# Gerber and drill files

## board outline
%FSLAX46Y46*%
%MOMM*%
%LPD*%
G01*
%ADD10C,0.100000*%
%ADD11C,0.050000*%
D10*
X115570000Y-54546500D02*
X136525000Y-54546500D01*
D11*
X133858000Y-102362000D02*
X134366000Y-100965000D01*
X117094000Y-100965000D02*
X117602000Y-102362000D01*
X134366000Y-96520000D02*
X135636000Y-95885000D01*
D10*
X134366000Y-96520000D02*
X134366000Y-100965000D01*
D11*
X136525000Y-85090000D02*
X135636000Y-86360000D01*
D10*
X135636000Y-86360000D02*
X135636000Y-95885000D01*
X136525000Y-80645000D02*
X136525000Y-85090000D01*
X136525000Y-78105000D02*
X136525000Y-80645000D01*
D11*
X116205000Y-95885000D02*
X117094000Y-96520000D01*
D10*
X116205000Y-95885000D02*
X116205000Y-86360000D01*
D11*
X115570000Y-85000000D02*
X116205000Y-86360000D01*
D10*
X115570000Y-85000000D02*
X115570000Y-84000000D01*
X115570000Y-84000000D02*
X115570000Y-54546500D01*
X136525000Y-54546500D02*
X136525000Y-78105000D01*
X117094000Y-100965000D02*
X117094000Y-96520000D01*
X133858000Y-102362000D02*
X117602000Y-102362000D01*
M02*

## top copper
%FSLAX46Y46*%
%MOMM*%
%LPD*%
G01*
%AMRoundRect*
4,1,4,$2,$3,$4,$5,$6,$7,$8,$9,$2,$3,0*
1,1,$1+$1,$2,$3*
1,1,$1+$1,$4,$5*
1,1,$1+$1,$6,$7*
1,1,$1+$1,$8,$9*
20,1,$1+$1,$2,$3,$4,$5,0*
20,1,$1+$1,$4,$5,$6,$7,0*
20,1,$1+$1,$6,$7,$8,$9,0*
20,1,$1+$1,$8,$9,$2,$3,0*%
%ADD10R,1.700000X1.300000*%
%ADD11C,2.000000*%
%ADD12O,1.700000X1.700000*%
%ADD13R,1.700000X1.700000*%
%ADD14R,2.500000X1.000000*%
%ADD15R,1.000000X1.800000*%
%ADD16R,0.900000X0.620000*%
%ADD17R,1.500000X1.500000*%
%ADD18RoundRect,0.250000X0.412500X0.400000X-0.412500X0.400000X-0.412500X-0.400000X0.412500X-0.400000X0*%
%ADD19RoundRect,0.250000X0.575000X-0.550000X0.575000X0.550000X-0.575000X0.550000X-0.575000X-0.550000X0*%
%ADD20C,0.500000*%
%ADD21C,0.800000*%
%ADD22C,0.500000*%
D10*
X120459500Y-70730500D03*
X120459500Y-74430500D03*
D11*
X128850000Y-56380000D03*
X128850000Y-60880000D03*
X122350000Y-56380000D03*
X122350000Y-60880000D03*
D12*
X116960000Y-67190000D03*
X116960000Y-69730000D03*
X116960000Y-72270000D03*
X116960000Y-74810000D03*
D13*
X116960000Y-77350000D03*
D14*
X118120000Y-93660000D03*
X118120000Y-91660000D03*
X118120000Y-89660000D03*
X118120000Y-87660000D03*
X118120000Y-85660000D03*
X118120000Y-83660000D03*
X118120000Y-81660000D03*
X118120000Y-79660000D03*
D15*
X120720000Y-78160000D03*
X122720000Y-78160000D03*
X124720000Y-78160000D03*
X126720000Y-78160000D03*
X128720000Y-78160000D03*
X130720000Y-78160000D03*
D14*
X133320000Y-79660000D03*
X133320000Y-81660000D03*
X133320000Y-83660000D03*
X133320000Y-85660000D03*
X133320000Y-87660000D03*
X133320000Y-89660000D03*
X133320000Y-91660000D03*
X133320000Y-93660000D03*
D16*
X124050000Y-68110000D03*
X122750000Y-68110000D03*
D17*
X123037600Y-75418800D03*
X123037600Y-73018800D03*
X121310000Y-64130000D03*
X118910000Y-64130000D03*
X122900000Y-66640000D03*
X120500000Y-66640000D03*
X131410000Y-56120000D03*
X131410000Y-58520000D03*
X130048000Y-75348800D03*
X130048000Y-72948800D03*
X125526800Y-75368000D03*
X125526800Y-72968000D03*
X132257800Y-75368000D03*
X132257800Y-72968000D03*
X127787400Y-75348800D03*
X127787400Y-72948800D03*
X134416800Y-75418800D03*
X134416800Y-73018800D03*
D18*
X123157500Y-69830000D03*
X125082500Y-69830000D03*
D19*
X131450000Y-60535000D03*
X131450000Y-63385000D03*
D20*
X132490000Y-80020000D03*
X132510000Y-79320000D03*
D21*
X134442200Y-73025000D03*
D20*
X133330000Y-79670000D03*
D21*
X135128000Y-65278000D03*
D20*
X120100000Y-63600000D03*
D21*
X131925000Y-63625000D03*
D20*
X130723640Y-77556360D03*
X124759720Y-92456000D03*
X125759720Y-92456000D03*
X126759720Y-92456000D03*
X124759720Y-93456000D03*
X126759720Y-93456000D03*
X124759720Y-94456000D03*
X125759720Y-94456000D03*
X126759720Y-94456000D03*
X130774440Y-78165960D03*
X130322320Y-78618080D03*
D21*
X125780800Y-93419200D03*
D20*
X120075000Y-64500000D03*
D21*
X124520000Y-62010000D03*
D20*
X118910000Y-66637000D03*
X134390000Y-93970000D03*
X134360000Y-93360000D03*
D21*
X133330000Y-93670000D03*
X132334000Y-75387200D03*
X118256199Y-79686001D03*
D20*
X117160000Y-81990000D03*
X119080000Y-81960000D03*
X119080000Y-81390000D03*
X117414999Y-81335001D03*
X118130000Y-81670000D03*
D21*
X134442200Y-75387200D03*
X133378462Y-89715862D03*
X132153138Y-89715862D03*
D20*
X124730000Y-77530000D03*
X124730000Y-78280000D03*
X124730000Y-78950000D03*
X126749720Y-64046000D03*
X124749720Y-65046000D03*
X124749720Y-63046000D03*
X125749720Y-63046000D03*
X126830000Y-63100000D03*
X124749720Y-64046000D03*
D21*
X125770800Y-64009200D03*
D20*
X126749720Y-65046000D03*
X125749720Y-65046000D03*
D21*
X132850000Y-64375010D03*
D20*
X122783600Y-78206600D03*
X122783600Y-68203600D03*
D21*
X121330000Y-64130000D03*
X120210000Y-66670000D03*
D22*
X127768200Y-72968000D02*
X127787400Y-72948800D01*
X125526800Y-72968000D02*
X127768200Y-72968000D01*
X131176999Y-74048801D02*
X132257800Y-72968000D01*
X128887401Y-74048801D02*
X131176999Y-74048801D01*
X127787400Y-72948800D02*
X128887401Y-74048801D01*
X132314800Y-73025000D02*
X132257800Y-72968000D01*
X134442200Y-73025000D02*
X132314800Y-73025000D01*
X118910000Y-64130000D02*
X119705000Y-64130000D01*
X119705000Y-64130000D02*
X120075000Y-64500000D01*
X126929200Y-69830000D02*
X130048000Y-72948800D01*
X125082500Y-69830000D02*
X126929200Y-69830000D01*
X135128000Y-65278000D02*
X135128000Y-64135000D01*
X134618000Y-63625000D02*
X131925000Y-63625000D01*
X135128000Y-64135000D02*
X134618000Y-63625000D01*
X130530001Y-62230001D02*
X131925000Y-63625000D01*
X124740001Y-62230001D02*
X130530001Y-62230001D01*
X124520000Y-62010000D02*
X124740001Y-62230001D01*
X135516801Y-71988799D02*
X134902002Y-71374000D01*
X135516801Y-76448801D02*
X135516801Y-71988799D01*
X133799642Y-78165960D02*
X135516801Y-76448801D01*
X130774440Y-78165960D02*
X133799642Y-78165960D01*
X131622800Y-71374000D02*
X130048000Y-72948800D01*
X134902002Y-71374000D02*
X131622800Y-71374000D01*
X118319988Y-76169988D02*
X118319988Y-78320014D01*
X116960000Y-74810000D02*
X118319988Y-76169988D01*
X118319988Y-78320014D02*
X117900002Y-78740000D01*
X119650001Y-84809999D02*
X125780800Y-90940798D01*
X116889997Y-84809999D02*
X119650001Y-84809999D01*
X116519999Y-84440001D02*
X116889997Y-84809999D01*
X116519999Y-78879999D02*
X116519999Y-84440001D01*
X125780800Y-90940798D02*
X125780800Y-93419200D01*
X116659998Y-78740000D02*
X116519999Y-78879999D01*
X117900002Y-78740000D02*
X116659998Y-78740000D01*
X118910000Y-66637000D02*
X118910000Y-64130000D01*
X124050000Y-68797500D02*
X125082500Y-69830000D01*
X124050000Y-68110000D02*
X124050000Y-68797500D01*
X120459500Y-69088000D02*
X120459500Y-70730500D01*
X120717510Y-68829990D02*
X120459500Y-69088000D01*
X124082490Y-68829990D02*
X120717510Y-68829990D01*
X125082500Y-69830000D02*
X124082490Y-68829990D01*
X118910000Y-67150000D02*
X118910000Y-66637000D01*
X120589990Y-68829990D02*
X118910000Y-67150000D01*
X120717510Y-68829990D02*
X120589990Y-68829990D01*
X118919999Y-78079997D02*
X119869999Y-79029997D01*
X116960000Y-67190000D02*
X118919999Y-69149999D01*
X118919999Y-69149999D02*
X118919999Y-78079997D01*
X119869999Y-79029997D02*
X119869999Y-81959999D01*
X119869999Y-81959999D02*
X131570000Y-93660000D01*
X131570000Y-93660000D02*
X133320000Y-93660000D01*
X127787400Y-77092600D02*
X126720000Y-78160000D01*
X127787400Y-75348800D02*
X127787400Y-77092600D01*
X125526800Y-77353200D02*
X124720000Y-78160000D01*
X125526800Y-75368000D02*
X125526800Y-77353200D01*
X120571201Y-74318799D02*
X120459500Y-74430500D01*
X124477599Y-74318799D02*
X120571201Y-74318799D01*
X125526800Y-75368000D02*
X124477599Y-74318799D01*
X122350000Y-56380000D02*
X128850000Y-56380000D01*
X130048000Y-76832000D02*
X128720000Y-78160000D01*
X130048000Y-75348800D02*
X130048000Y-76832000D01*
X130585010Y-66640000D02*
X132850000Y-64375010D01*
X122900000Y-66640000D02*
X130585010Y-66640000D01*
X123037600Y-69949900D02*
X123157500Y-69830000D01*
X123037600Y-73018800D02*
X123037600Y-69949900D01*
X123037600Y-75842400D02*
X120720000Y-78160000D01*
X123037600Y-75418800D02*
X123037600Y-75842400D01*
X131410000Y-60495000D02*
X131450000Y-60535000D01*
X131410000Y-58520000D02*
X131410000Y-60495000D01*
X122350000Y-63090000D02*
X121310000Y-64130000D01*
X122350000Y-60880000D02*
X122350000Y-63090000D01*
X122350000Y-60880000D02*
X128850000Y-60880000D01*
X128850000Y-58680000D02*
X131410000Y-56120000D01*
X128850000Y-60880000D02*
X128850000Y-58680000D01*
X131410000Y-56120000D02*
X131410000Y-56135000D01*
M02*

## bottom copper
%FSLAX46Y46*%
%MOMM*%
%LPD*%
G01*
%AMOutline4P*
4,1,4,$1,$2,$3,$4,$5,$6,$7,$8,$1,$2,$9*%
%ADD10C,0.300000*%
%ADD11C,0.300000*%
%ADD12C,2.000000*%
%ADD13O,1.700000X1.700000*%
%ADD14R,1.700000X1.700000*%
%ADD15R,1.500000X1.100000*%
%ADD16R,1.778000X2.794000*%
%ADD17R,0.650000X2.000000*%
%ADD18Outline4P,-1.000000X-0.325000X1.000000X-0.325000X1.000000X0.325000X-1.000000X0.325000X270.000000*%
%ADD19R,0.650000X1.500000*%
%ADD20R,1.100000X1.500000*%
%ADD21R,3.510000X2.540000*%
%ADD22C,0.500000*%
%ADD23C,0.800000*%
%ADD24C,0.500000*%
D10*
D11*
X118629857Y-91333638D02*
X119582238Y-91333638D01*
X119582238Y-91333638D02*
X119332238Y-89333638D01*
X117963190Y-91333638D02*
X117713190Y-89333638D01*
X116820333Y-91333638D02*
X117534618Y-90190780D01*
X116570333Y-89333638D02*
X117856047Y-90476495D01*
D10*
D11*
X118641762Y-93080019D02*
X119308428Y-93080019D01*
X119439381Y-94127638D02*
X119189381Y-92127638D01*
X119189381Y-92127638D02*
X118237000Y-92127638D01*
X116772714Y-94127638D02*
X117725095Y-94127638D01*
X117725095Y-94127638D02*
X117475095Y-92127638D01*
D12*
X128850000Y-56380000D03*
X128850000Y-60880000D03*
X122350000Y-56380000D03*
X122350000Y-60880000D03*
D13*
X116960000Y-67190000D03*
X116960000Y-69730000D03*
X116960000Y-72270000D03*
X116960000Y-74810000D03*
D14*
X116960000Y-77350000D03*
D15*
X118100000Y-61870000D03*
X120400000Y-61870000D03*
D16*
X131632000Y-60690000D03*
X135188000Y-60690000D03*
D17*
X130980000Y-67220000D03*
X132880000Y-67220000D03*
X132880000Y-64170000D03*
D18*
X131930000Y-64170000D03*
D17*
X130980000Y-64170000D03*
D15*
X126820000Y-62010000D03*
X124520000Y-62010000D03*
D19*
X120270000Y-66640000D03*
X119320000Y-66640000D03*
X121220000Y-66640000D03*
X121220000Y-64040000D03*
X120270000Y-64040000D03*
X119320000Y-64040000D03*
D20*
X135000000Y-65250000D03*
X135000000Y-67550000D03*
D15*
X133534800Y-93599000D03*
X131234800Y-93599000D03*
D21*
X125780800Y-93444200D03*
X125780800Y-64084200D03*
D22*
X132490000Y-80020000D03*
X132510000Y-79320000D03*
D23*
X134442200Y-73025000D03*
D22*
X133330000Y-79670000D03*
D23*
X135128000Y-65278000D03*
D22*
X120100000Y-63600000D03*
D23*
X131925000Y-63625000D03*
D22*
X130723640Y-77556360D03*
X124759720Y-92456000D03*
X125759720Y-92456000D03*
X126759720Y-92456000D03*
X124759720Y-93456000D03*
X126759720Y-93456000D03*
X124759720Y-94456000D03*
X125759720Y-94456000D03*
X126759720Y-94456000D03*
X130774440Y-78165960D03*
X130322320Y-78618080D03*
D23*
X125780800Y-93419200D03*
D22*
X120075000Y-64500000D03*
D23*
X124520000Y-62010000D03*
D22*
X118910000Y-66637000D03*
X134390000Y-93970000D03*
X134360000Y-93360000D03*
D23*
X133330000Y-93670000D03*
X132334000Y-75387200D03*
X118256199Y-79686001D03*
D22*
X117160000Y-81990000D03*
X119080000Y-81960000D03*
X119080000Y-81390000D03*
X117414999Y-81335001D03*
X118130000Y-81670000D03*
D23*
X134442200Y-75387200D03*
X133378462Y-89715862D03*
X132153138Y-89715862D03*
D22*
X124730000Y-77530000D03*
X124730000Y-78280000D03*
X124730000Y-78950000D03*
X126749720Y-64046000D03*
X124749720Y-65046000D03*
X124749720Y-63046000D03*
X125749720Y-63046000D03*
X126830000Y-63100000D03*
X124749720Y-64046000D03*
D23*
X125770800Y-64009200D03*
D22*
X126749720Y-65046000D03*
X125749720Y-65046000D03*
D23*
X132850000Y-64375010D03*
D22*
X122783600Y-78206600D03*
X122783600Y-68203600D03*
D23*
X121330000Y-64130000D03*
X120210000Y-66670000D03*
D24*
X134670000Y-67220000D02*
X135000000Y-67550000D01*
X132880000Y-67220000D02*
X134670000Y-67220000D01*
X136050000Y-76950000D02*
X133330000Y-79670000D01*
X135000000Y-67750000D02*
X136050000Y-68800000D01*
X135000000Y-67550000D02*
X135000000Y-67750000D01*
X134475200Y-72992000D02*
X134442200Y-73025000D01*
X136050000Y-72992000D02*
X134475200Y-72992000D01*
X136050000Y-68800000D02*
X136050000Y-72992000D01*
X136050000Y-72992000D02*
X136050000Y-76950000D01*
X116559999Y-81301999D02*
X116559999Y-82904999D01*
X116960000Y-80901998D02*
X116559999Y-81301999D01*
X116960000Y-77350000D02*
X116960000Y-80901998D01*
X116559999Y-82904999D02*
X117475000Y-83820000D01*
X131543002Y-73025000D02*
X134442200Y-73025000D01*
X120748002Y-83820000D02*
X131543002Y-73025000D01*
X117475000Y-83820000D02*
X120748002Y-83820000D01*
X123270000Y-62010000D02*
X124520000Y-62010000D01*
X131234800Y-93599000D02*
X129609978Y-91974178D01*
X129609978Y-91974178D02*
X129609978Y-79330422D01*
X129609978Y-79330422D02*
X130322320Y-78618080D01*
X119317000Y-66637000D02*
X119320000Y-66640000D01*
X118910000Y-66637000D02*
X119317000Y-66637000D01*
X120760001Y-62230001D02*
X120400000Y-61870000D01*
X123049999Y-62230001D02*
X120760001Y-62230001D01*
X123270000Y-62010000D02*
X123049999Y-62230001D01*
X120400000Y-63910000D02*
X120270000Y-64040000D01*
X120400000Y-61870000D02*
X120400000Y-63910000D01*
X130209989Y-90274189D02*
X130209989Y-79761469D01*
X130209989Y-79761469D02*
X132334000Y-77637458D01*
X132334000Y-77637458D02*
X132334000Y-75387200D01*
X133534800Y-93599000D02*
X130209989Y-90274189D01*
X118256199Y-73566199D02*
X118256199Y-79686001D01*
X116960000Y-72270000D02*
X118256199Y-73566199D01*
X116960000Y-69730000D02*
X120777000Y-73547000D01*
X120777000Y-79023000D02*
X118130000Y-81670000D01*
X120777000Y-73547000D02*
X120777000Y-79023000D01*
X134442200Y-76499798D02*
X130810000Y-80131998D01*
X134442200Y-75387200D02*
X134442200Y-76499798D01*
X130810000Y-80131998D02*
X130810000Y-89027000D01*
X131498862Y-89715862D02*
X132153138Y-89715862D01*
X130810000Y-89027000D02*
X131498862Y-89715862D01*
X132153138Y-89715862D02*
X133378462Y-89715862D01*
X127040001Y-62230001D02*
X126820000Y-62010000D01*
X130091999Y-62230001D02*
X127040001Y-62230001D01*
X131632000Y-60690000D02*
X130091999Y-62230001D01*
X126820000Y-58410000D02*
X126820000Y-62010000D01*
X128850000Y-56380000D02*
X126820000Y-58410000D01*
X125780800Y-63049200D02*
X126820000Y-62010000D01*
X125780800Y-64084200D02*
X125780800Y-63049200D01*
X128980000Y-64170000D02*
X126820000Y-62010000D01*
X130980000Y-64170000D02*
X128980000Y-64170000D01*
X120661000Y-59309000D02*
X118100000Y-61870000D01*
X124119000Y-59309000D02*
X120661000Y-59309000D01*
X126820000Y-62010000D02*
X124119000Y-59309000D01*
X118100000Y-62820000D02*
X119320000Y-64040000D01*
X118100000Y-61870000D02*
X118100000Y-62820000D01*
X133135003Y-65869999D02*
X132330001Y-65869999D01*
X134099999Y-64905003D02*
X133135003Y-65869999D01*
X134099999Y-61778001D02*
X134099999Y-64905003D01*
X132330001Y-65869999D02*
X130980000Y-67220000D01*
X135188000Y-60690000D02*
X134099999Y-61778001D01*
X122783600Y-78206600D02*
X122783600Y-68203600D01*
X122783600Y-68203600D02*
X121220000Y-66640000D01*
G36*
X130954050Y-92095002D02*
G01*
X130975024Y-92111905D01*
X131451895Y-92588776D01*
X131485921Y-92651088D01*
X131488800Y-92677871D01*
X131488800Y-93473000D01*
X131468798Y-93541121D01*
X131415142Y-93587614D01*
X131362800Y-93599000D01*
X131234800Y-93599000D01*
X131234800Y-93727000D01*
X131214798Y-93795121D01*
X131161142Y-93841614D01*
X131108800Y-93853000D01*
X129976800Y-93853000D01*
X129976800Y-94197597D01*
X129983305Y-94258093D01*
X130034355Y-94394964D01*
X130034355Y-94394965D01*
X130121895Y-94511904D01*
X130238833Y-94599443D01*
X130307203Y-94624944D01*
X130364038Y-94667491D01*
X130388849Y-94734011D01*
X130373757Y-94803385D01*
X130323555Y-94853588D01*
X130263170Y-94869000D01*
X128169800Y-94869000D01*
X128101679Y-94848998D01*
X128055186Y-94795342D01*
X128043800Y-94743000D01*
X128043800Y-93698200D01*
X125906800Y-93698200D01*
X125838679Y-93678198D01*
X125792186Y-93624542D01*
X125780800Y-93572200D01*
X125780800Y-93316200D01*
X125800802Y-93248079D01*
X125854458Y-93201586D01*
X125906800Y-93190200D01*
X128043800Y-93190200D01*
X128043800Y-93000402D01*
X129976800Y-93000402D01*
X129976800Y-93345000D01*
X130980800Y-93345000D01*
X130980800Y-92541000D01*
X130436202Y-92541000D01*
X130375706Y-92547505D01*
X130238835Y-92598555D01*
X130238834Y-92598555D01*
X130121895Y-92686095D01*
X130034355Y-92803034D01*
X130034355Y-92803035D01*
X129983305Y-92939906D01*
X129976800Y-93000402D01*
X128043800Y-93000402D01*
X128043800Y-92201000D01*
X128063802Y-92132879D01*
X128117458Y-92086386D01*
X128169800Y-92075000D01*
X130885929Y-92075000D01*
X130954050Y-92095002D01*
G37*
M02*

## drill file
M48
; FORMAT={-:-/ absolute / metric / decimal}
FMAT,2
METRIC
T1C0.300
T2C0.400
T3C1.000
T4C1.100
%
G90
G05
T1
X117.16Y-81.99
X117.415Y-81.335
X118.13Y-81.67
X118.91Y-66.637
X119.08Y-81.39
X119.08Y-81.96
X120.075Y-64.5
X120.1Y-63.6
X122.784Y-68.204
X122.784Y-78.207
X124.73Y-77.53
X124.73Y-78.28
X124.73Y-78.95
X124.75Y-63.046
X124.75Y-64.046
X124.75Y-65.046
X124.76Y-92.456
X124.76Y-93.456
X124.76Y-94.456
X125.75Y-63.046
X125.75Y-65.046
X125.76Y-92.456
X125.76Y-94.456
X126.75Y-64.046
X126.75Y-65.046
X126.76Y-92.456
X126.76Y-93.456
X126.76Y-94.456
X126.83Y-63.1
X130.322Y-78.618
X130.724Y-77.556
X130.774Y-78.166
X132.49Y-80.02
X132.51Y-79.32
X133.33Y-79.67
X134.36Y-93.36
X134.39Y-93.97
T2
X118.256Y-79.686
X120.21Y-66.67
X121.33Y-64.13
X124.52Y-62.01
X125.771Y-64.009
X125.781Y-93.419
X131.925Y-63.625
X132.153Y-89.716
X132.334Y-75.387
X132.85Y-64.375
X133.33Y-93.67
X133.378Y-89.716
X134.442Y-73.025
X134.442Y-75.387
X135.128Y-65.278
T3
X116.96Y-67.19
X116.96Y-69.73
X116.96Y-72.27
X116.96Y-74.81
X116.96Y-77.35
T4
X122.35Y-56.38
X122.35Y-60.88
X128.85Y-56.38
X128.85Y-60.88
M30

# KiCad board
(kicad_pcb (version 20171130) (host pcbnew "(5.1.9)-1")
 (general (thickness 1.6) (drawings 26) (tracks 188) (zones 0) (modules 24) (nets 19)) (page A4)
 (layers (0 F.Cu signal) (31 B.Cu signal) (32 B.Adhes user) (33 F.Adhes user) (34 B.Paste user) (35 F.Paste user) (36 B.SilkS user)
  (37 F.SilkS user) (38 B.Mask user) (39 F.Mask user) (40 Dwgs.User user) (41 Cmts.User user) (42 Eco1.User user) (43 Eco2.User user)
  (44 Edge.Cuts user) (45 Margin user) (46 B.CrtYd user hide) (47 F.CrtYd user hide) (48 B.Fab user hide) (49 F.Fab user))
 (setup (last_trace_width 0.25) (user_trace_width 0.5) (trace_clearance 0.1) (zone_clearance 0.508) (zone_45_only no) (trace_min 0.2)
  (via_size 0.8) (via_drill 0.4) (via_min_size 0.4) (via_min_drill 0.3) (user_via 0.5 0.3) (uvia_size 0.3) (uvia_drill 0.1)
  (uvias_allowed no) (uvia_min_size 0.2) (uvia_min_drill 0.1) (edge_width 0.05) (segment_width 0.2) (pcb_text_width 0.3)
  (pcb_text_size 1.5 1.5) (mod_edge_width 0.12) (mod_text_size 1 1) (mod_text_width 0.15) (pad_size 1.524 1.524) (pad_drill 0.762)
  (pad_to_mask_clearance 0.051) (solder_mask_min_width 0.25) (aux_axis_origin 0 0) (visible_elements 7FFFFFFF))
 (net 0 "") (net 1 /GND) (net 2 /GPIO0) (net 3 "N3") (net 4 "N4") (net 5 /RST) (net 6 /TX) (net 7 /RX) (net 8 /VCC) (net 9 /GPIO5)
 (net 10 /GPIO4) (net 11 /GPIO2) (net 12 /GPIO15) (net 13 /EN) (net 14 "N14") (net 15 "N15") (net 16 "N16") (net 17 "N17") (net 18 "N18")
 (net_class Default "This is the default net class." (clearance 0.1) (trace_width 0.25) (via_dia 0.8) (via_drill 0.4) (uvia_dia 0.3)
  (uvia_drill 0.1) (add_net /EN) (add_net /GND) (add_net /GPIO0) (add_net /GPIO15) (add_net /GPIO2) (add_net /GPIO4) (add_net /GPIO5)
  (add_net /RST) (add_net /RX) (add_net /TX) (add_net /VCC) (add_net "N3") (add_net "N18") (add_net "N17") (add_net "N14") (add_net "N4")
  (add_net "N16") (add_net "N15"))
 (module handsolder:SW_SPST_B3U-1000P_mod (layer F.Cu) (at 120.4595 72.5805 90)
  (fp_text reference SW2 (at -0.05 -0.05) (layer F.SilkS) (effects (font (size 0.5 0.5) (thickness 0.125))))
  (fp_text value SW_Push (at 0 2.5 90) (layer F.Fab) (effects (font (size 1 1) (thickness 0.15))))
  (pad 2 smd rect (at 1.85 0 90) (size 1.3 1.7) (layers F.Cu F.Paste F.Mask) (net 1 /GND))
  (pad 1 smd rect (at -1.85 0 90) (size 1.3 1.7) (layers F.Cu F.Paste F.Mask) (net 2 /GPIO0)))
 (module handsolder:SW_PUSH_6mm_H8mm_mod (layer F.Cu) (at 122.35 56.38)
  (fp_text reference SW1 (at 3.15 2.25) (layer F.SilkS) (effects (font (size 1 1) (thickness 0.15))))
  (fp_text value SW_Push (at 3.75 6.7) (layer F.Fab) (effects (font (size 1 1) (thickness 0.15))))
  (pad 1 thru_hole circle (at 6.5 0 90) (size 2 2) (drill 1.1) (layers *.Cu *.Mask) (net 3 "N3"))
  (pad 2 thru_hole circle (at 6.5 4.5 90) (size 2 2) (drill 1.1) (layers *.Cu *.Mask) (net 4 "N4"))
  (pad 1 thru_hole circle (at 0 0 90) (size 2 2) (drill 1.1) (layers *.Cu *.Mask) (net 3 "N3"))
  (pad 2 thru_hole circle (at 0 4.5 90) (size 2 2) (drill 1.1) (layers *.Cu *.Mask) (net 4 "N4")))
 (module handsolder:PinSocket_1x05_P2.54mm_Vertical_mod (layer F.Cu) (at 116.96 77.35 180)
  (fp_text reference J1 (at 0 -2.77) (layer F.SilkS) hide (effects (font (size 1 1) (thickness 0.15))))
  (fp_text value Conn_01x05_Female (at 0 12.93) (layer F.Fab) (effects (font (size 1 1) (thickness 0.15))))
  (pad 5 thru_hole oval (at 0 10.16 180) (size 1.7 1.7) (drill 1) (layers *.Cu *.Mask) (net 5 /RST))
  (pad 4 thru_hole oval (at 0 7.62 180) (size 1.7 1.7) (drill 1) (layers *.Cu *.Mask) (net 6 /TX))
  (pad 3 thru_hole oval (at 0 5.08 180) (size 1.7 1.7) (drill 1) (layers *.Cu *.Mask) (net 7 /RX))
  (pad 2 thru_hole oval (at 0 2.54 180) (size 1.7 1.7) (drill 1) (layers *.Cu *.Mask) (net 1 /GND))
  (pad 1 thru_hole rect (at 0 0 180) (size 1.7 1.7) (drill 1) (layers *.Cu *.Mask) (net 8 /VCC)))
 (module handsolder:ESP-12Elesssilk (layer F.Cu) (at 125.72 90.16 180)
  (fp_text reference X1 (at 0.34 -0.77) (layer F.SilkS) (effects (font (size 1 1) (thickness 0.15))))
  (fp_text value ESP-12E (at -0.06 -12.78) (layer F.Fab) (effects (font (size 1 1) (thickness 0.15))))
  (pad 22 smd rect (at 7.6 -3.5 180) (size 2.5 1) (layers F.Cu F.Paste F.Mask))
  (pad 21 smd rect (at 7.6 -1.5 180) (size 2.5 1) (layers F.Cu F.Paste F.Mask))
  (pad 20 smd rect (at 7.6 0.5 180) (size 2.5 1) (layers F.Cu F.Paste F.Mask))
  (pad 19 smd rect (at 7.6 2.5 180) (size 2.5 1) (layers F.Cu F.Paste F.Mask))
  (pad 18 smd rect (at 7.6 4.5 180) (size 2.5 1) (layers F.Cu F.Paste F.Mask))
  (pad 17 smd rect (at 7.6 6.5 180) (size 2.5 1) (layers F.Cu F.Paste F.Mask))
  (pad 16 smd rect (at 7.6 8.5 180) (size 2.5 1) (layers F.Cu F.Paste F.Mask) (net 6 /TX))
  (pad 15 smd rect (at 7.6 10.5 180) (size 2.5 1) (layers F.Cu F.Paste F.Mask) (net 7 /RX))
  (pad 14 smd rect (at 5 12 180) (size 1 1.8) (layers F.Cu F.Paste F.Mask) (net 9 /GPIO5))
  (pad 13 smd rect (at 3 12 180) (size 1 1.8) (layers F.Cu F.Paste F.Mask) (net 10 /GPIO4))
  (pad 12 smd rect (at 1 12 180) (size 1 1.8) (layers F.Cu F.Paste F.Mask) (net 2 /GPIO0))
  (pad 11 smd rect (at -1 12 180) (size 1 1.8) (layers F.Cu F.Paste F.Mask) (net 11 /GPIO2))
  (pad 10 smd rect (at -3 12 180) (size 1 1.8) (layers F.Cu F.Paste F.Mask) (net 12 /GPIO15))
  (pad 9 smd rect (at -5 12 180) (size 1 1.8) (layers F.Cu F.Paste F.Mask) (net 1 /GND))
  (pad 8 smd rect (at -7.6 10.5 180) (size 2.5 1) (layers F.Cu F.Paste F.Mask) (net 8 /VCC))
  (pad 7 smd rect (at -7.6 8.5 180) (size 2.5 1) (layers F.Cu F.Paste F.Mask))
  (pad 6 smd rect (at -7.6 6.5 180) (size 2.5 1) (layers F.Cu F.Paste F.Mask))
  (pad 5 smd rect (at -7.6 4.5 180) (size 2.5 1) (layers F.Cu F.Paste F.Mask))
  (pad 4 smd rect (at -7.6 2.5 180) (size 2.5 1) (layers F.Cu F.Paste F.Mask))
  (pad 3 smd rect (at -7.6 0.5 180) (size 2.5 1) (layers F.Cu F.Paste F.Mask) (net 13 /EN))
  (pad 2 smd rect (at -7.6 -1.5 180) (size 2.5 1) (layers F.Cu F.Paste F.Mask))
  (pad 1 smd rect (at -7.6 -3.5 180) (size 2.5 1) (layers F.Cu F.Paste F.Mask) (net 5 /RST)))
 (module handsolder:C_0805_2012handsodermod (layer B.Cu) (at 119.25 61.87 180)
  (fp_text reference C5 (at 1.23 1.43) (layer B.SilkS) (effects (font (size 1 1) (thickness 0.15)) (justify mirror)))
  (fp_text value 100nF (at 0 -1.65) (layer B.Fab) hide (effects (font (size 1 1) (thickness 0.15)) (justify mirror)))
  (pad 2 smd rect (at 1.15 0 180) (size 1.5 1.1) (layers B.Cu B.Paste B.Mask) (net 3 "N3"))
  (pad 1 smd rect (at -1.15 0 180) (size 1.5 1.1) (layers B.Cu B.Paste B.Mask) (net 1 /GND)))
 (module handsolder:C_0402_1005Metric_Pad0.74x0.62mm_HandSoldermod (layer F.Cu) (at 123.4 68.11)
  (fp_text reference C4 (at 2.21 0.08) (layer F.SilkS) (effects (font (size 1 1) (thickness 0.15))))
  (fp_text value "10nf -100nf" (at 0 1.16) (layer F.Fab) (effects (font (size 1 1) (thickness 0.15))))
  (pad 2 smd rect (at 0.65 0) (size 0.9 0.62) (layers F.Cu F.Paste F.Mask) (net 1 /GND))
  (pad 1 smd rect (at -0.65 0) (size 0.9 0.62) (layers F.Cu F.Paste F.Mask) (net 10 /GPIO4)))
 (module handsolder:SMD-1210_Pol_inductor (layer B.Cu) (at 133.41 60.69)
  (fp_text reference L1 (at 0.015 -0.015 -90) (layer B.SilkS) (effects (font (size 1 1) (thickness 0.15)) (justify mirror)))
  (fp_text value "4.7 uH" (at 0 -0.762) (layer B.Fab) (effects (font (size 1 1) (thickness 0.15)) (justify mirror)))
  (pad 1 smd rect (at -1.778 0) (size 1.778 2.794) (layers B.Cu B.Paste B.Mask) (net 3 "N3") (zone_connect 2))
  (pad 2 smd rect (at 1.778 0) (size 1.778 2.794) (layers B.Cu B.Paste B.Mask) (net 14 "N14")))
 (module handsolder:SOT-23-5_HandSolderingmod (layer B.Cu) (at 131.93 65.72 270)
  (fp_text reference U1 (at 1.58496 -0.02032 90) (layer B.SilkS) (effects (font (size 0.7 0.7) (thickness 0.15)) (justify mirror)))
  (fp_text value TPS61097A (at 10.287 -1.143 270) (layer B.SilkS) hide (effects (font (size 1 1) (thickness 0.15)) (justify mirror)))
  (pad 5 smd rect (at 1.5 0.95 270) (size 2 0.65) (layers B.Cu B.Paste B.Mask) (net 14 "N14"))
  (pad 4 smd rect (at 1.5 -0.95 270) (size 2 0.65) (layers B.Cu B.Paste B.Mask) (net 8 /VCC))
  (pad 3 smd rect (at -1.55 -0.95 270) (size 2 0.65) (layers B.Cu B.Paste B.Mask) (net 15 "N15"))
  (pad 2 smd trapezoid (at -1.55 0 270) (size 2 0.65) (layers B.Cu B.Paste B.Mask) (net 1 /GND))
  (pad 1 smd rect (at -1.55 0.95 270) (size 2 0.65) (layers B.Cu B.Paste B.Mask) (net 3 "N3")))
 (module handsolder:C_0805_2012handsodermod (layer B.Cu) (at 125.67 62.01)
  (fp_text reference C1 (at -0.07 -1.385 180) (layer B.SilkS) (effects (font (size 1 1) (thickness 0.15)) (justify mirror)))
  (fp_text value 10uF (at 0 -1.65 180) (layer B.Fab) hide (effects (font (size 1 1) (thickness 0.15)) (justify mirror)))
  (pad 2 smd rect (at 1.15 0) (size 1.5 1.1) (layers B.Cu B.Paste B.Mask) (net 3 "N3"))
  (pad 1 smd rect (at -1.15 0) (size 1.5 1.1) (layers B.Cu B.Paste B.Mask) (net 1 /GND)))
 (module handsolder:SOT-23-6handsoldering (layer B.Cu) (at 120.27 65.34 270)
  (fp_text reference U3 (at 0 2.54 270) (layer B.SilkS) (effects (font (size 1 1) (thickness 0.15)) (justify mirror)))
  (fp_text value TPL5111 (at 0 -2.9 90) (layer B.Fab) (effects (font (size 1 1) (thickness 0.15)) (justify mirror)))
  (pad 5 smd rect (at 1.3 0 270) (size 1.5 0.65) (layers B.Cu B.Paste B.Mask) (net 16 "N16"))
  (pad 6 smd rect (at 1.3 0.95 270) (size 1.5 0.65) (layers B.Cu B.Paste B.Mask) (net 1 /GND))
  (pad 4 smd rect (at 1.3 -0.95 270) (size 1.5 0.65) (layers B.Cu B.Paste B.Mask) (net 10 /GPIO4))
  (pad 3 smd rect (at -1.3 -0.95 270) (size 1.5 0.65) (layers B.Cu B.Paste B.Mask) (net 4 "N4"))
  (pad 2 smd rect (at -1.3 0 270) (size 1.5 0.65) (layers B.Cu B.Paste B.Mask) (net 1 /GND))
  (pad 1 smd rect (at -1.3 0.95 270) (size 1.5 0.65) (layers B.Cu B.Paste B.Mask) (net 3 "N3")))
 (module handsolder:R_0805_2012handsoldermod (layer F.Cu) (at 123.0376 74.2188 270)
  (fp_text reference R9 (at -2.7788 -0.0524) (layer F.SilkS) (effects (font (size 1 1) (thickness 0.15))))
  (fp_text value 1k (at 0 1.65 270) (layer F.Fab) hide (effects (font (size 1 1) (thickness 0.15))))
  (pad 2 smd rect (at 1.2 0 270) (size 1.5 1.5) (layers F.Cu F.Paste F.Mask) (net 9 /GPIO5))
  (pad 1 smd rect (at -1.2 0 270) (size 1.5 1.5) (layers F.Cu F.Paste F.Mask) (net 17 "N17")))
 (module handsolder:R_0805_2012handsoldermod (layer F.Cu) (at 120.11 64.13)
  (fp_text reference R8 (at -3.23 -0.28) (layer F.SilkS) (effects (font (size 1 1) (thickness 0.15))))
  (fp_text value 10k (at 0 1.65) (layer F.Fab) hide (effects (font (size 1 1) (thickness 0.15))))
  (pad 2 smd rect (at 1.2 0) (size 1.5 1.5) (layers F.Cu F.Paste F.Mask) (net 4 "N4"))
  (pad 1 smd rect (at -1.2 0) (size 1.5 1.5) (layers F.Cu F.Paste F.Mask) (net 1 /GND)))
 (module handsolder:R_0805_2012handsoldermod (layer F.Cu) (at 121.7 66.64)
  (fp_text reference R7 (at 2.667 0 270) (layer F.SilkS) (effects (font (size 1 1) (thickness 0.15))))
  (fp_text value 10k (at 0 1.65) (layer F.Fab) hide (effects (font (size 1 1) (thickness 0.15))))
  (pad 2 smd rect (at 1.2 0) (size 1.5 1.5) (layers F.Cu F.Paste F.Mask) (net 15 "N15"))
  (pad 1 smd rect (at -1.2 0) (size 1.5 1.5) (layers F.Cu F.Paste F.Mask) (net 16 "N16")))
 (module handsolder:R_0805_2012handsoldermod (layer F.Cu) (at 131.41 57.32 90)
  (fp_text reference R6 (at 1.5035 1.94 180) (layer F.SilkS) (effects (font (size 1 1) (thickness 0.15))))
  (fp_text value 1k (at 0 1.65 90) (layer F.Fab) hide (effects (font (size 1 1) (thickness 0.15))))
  (pad 2 smd rect (at 1.2 0 90) (size 1.5 1.5) (layers F.Cu F.Paste F.Mask) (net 4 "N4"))
  (pad 1 smd rect (at -1.2 0 90) (size 1.5 1.5) (layers F.Cu F.Paste F.Mask) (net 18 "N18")))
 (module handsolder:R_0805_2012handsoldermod (layer F.Cu) (at 130.048 74.1488 270)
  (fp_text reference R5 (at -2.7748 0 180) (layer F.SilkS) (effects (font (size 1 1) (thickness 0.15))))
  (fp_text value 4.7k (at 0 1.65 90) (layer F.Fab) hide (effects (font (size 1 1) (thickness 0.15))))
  (pad 2 smd rect (at 1.2 0 270) (size 1.5 1.5) (layers F.Cu F.Paste F.Mask) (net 12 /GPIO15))
  (pad 1 smd rect (at -1.2 0 270) (size 1.5 1.5) (layers F.Cu F.Paste F.Mask) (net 1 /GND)))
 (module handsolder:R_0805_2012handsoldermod (layer F.Cu) (at 125.5268 74.168 270)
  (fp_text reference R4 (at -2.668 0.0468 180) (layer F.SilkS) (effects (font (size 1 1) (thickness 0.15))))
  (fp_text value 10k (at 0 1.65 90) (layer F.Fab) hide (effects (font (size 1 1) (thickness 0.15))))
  (pad 2 smd rect (at 1.2 0 270) (size 1.5 1.5) (layers F.Cu F.Paste F.Mask) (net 2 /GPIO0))
  (pad 1 smd rect (at -1.2 0 270) (size 1.5 1.5) (layers F.Cu F.Paste F.Mask) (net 8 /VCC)))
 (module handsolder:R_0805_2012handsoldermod (layer F.Cu) (at 132.2578 74.168 270)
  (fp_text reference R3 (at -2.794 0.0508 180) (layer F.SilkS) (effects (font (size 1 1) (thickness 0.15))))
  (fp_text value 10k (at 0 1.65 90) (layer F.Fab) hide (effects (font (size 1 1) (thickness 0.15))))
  (pad 2 smd rect (at 1.2 0 270) (size 1.5 1.5) (layers F.Cu F.Paste F.Mask) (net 5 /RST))
  (pad 1 smd rect (at -1.2 0 270) (size 1.5 1.5) (layers F.Cu F.Paste F.Mask) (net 8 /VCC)))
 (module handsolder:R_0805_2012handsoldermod (layer F.Cu) (at 127.7874 74.1488 270)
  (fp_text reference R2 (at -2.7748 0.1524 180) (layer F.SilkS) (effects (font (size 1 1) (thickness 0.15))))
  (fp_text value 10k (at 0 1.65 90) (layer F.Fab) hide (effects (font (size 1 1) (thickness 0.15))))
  (pad 2 smd rect (at 1.2 0 270) (size 1.5 1.5) (layers F.Cu F.Paste F.Mask) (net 11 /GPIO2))
  (pad 1 smd rect (at -1.2 0 270) (size 1.5 1.5) (layers F.Cu F.Paste F.Mask) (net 8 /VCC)))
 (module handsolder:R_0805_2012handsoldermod (layer F.Cu) (at 134.4168 74.2188 270)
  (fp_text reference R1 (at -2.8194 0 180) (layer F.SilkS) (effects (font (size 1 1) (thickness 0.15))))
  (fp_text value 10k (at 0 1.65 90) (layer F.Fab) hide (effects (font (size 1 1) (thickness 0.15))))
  (pad 2 smd rect (at 1.2 0 270) (size 1.5 1.5) (layers F.Cu F.Paste F.Mask) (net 13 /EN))
  (pad 1 smd rect (at -1.2 0 270) (size 1.5 1.5) (layers F.Cu F.Paste F.Mask) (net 8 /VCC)))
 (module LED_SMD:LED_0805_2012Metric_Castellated (layer F.Cu) (at 124.12 69.83 180)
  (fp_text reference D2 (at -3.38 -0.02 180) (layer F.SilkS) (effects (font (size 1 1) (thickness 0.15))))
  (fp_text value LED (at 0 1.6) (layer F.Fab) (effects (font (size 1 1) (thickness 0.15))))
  (pad 2 smd roundrect (at 0.9625 0 180) (size 1.325 1.3) (layers F.Cu F.Paste F.Mask) (roundrect_rratio 0.1923076923076923) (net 17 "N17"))
  (pad 1 smd roundrect (at -0.9625 0 180) (size 1.325 1.3) (layers F.Cu F.Paste F.Mask) (roundrect_rratio 0.1923076923076923) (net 1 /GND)))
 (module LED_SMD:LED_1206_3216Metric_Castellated (layer F.Cu) (at 131.45 61.96 90)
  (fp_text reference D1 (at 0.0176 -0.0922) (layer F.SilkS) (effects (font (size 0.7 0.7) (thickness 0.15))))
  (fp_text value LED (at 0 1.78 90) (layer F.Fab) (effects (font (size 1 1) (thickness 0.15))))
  (pad 2 smd roundrect (at 1.425 0 90) (size 1.6 1.65) (layers F.Cu F.Paste F.Mask) (roundrect_rratio 0.15625) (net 18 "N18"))
  (pad 1 smd roundrect (at -1.425 0 90) (size 1.6 1.65) (layers F.Cu F.Paste F.Mask) (roundrect_rratio 0.15625) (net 1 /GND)))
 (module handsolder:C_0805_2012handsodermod (layer B.Cu) (at 135 66.4 90)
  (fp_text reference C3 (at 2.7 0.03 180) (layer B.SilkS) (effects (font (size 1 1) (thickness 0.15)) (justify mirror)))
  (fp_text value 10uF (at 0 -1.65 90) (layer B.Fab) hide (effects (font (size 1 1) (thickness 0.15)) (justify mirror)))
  (pad 2 smd rect (at 1.15 0 90) (size 1.5 1.1) (layers B.Cu B.Paste B.Mask) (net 1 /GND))
  (pad 1 smd rect (at -1.15 0 90) (size 1.5 1.1) (layers B.Cu B.Paste B.Mask) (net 8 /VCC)))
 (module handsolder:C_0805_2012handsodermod (layer B.Cu) (at 132.3848 93.599)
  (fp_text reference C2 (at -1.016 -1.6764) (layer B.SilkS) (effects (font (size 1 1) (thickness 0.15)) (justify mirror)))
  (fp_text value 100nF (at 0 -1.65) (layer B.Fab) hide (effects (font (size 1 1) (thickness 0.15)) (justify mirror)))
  (pad 2 smd rect (at 1.15 0) (size 1.5 1.1) (layers B.Cu B.Paste B.Mask) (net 5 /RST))
  (pad 1 smd rect (at -1.15 0) (size 1.5 1.1) (layers B.Cu B.Paste B.Mask) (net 1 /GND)))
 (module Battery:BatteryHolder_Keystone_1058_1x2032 (layer B.Cu) (at 125.7808 78.7642 270)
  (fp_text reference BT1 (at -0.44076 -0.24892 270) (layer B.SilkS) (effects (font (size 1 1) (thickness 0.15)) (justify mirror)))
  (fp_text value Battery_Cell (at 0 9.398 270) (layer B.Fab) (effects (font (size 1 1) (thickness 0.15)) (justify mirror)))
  (pad 2 smd rect (at 14.68 0 270) (size 2.54 3.51) (layers B.Cu B.Paste B.Mask) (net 1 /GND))
  (pad 1 smd rect (at -14.68 0 270) (size 2.54 3.51) (layers B.Cu B.Paste B.Mask) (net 3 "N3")))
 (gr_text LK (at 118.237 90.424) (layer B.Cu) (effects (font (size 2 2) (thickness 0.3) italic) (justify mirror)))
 (gr_line (start 115.57 54.5465) (end 136.525 54.5465) (layer Edge.Cuts) (width 0.1))
 (gr_line (start 133.858 102.362) (end 134.366 100.965) (layer Edge.Cuts) (width 0.05))
 (gr_line (start 117.094 100.965) (end 117.602 102.362) (layer Edge.Cuts) (width 0.05))
 (gr_line (start 134.366 96.52) (end 135.636 95.885) (layer Edge.Cuts) (width 0.05))
 (gr_line (start 134.366 96.52) (end 134.366 100.965) (layer Edge.Cuts) (width 0.1))
 (gr_line (start 136.525 85.09) (end 135.636 86.36) (layer Edge.Cuts) (width 0.05))
 (gr_line (start 135.636 86.36) (end 135.636 95.885) (layer Edge.Cuts) (width 0.1))
 (gr_line (start 136.525 80.645) (end 136.525 85.09) (layer Edge.Cuts) (width 0.1))
 (gr_line (start 136.525 78.105) (end 136.525 80.645) (layer Edge.Cuts) (width 0.1))
 (gr_line (start 116.205 95.885) (end 117.094 96.52) (layer Edge.Cuts) (width 0.05))
 (gr_line (start 116.205 95.885) (end 116.205 86.36) (layer Edge.Cuts) (width 0.1))
 (gr_line (start 115.57 85) (end 116.205 86.36) (layer Edge.Cuts) (width 0.05))
 (gr_line (start 115.57 85) (end 115.57 84) (layer Edge.Cuts) (width 0.1))
 (gr_line (start 115.57 84) (end 115.57 54.5465) (layer Edge.Cuts) (width 0.1))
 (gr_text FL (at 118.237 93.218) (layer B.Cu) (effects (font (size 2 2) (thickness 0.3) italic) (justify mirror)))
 (gr_line (start 136.525 54.5465) (end 136.525 78.105) (layer Edge.Cuts) (width 0.1))
 (gr_line (start 117.094 100.965) (end 117.094 96.52) (layer Edge.Cuts) (width 0.1))
 (gr_line (start 133.858 102.362) (end 117.602 102.362) (layer Edge.Cuts) (width 0.1))
 (via (at 132.49 80.02) (size 0.5) (drill 0.3) (layers F.Cu B.Cu) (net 8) (status 30))
 (via (at 132.51 79.32) (size 0.5) (drill 0.3) (layers F.Cu B.Cu) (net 8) (status 30))
 (via (at 134.4422 73.025) (size 0.8) (drill 0.4) (layers F.Cu B.Cu) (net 8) (status 30))
 (via (at 133.33 79.67) (size 0.5) (drill 0.3) (layers F.Cu B.Cu) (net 8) (status 30))
 (segment (start 127.7682 72.968) (end 127.7874 72.9488) (width 0.5) (layer F.Cu) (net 8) (status 30))
 (segment (start 125.5268 72.968) (end 127.7682 72.968) (width 0.5) (layer F.Cu) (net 8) (status 30))
 (segment (start 131.176999 74.048801) (end 132.2578 72.968) (width 0.5) (layer F.Cu) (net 8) (status 20))
 (segment (start 128.887401 74.048801) (end 131.176999 74.048801) (width 0.5) (layer F.Cu) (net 8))
 (segment (start 127.7874 72.9488) (end 128.887401 74.048801) (width 0.5) (layer F.Cu) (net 8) (status 10))
 (segment (start 134.67 67.22) (end 135 67.55) (width 0.5) (layer B.Cu) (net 8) (status 30))
 (segment (start 132.88 67.22) (end 134.67 67.22) (width 0.5) (layer B.Cu) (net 8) (status 30))
 (segment (start 136.05 76.95) (end 133.33 79.67) (width 0.5) (layer B.Cu) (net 8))
 (segment (start 135 67.75) (end 136.05 68.8) (width 0.5) (layer B.Cu) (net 8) (status 10))
 (segment (start 135 67.55) (end 135 67.75) (width 0.5) (layer B.Cu) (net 8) (status 30))
 (segment (start 134.4752 72.992) (end 134.4422 73.025) (width 0.5) (layer B.Cu) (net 8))
 (segment (start 136.05 72.992) (end 134.4752 72.992) (width 0.5) (layer B.Cu) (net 8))
 (segment (start 136.05 68.8) (end 136.05 72.992) (width 0.5) (layer B.Cu) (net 8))
 (segment (start 136.05 72.992) (end 136.05 76.95) (width 0.5) (layer B.Cu) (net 8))
 (segment (start 132.3148 73.025) (end 132.2578 72.968) (width 0.5) (layer F.Cu) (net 8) (status 30))
 (segment (start 134.4422 73.025) (end 132.3148 73.025) (width 0.5) (layer F.Cu) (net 8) (status 30))
 (segment (start 116.559999 81.301999) (end 116.559999 82.904999) (width 0.5) (layer B.Cu) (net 8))
 (segment (start 116.96 80.901998) (end 116.559999 81.301999) (width 0.5) (layer B.Cu) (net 8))
 (segment (start 116.96 77.35) (end 116.96 80.901998) (width 0.5) (layer B.Cu) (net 8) (status 10))
 (segment (start 116.559999 82.904999) (end 117.475 83.82) (width 0.5) (layer B.Cu) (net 8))
 (segment (start 131.543002 73.025) (end 134.4422 73.025) (width 0.5) (layer B.Cu) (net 8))
 (segment (start 120.748002 83.82) (end 131.543002 73.025) (width 0.5) (layer B.Cu) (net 8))
 (segment (start 117.475 83.82) (end 120.748002 83.82) (width 0.5) (layer B.Cu) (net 8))
 (via (at 135.128 65.278) (size 0.8) (drill 0.4) (layers F.Cu B.Cu) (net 1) (status 30))
 (via (at 120.1 63.6) (size 0.5) (drill 0.3) (layers F.Cu B.Cu) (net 1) (status 30))
 (via (at 131.925 63.625) (size 0.8) (drill 0.4) (layers F.Cu B.Cu) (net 1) (status 30))
 (via (at 130.72364 77.55636) (size 0.5) (drill 0.3) (layers F.Cu B.Cu) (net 1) (status 30))
 (via (at 124.75972 92.456) (size 0.5) (drill 0.3) (layers F.Cu B.Cu) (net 1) (status 30))
 (via (at 125.75972 92.456) (size 0.5) (drill 0.3) (layers F.Cu B.Cu) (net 1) (status 30))
 (via (at 126.75972 92.456) (size 0.5) (drill 0.3) (layers F.Cu B.Cu) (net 1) (status 30))
 (via (at 124.75972 93.456) (size 0.5) (drill 0.3) (layers F.Cu B.Cu) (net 1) (status 30))
 (via (at 126.75972 93.456) (size 0.5) (drill 0.3) (layers F.Cu B.Cu) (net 1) (status 30))
 (via (at 124.75972 94.456) (size 0.5) (drill 0.3) (layers F.Cu B.Cu) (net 1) (status 30))
 (via (at 125.75972 94.456) (size 0.5) (drill 0.3) (layers F.Cu B.Cu) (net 1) (status 30))
 (via (at 126.75972 94.456) (size 0.5) (drill 0.3) (layers F.Cu B.Cu) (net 1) (status 30))
 (via (at 130.77444 78.16596) (size 0.5) (drill 0.3) (layers F.Cu B.Cu) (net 1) (status 30))
 (via (at 130.32232 78.61808) (size 0.5) (drill 0.3) (layers F.Cu B.Cu) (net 1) (status 30))
 (via (at 125.7808 93.4192) (size 0.8) (drill 0.4) (layers F.Cu B.Cu) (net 1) (status 30))
 (segment (start 118.91 64.13) (end 119.705 64.13) (width 0.5) (layer F.Cu) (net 1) (status 10))
 (segment (start 119.705 64.13) (end 120.075 64.5) (width 0.5) (layer F.Cu) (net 1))
 (via (at 120.075 64.5) (size 0.5) (drill 0.3) (layers F.Cu B.Cu) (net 1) (status 30))
 (segment (start 126.9292 69.83) (end 130.048 72.9488) (width 0.5) (layer F.Cu) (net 1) (status 20))
 (segment (start 125.0825 69.83) (end 126.9292 69.83) (width 0.5) (layer F.Cu) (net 1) (status 10))
 (segment (start 123.27 62.01) (end 124.52 62.01) (width 0.5) (layer B.Cu) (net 1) (status 20))
 (segment (start 135.128 65.278) (end 135.128 64.135) (width 0.5) (layer F.Cu) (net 1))
 (segment (start 134.618 63.625) (end 131.925 63.625) (width 0.5) (layer F.Cu) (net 1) (status 20))
 (segment (start 135.128 64.135) (end 134.618 63.625) (width 0.5) (layer F.Cu) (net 1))
 (segment (start 131.2348 93.599) (end 129.609978 91.974178) (width 0.5) (layer B.Cu) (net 1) (status 10))
 (segment (start 129.609978 91.974178) (end 129.609978 79.330422) (width 0.5) (layer B.Cu) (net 1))
 (segment (start 129.609978 79.330422) (end 130.32232 78.61808) (width 0.5) (layer B.Cu) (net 1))
 (via (at 124.52 62.01) (size 0.8) (drill 0.4) (layers F.Cu B.Cu) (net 1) (status 30))
 (segment (start 130.530001 62.230001) (end 131.925 63.625) (width 0.5) (layer F.Cu) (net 1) (status 20))
 (segment (start 124.740001 62.230001) (end 130.530001 62.230001) (width 0.5) (layer F.Cu) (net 1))
 (segment (start 124.52 62.01) (end 124.740001 62.230001) (width 0.5) (layer F.Cu) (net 1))
 (segment (start 135.516801 71.988799) (end 134.902002 71.374) (width 0.5) (layer F.Cu) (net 1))
 (segment (start 135.516801 76.448801) (end 135.516801 71.988799) (width 0.5) (layer F.Cu) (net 1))
 (segment (start 133.799642 78.16596) (end 135.516801 76.448801) (width 0.5) (layer F.Cu) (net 1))
 (segment (start 130.77444 78.16596) (end 133.799642 78.16596) (width 0.5) (layer F.Cu) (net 1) (status 10))
 (segment (start 131.6228 71.374) (end 130.048 72.9488) (width 0.5) (layer F.Cu) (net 1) (status 20))
 (segment (start 134.902002 71.374) (end 131.6228 71.374) (width 0.5) (layer F.Cu) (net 1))
 (segment (start 118.319988 76.169988) (end 118.319988 78.320014) (width 0.5) (layer F.Cu) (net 1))
 (segment (start 116.96 74.81) (end 118.319988 76.169988) (width 0.5) (layer F.Cu) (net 1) (status 10))
 (segment (start 118.319988 78.320014) (end 117.900002 78.74) (width 0.5) (layer F.Cu) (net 1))
 (segment (start 119.650001 84.809999) (end 125.7808 90.940798) (width 0.5) (layer F.Cu) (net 1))
 (segment (start 116.889997 84.809999) (end 119.650001 84.809999) (width 0.5) (layer F.Cu) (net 1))
 (segment (start 116.519999 84.440001) (end 116.889997 84.809999) (width 0.5) (layer F.Cu) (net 1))
 (segment (start 116.519999 78.879999) (end 116.519999 84.440001) (width 0.5) (layer F.Cu) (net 1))
 (segment (start 125.7808 90.940798) (end 125.7808 93.4192) (width 0.5) (layer F.Cu) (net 1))
 (segment (start 116.659998 78.74) (end 116.519999 78.879999) (width 0.5) (layer F.Cu) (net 1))
 (segment (start 117.900002 78.74) (end 116.659998 78.74) (width 0.5) (layer F.Cu) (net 1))
 (segment (start 118.91 66.637) (end 118.91 64.13) (width 0.5) (layer F.Cu) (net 1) (status 20))
 (via (at 118.91 66.637) (size 0.5) (drill 0.3) (layers F.Cu B.Cu) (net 1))
 (segment (start 119.317 66.637) (end 119.32 66.64) (width 0.5) (layer B.Cu) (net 1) (status 30))
 (segment (start 118.91 66.637) (end 119.317 66.637) (width 0.5) (layer B.Cu) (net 1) (status 20))
 (segment (start 124.05 68.7975) (end 125.0825 69.83) (width 0.5) (layer F.Cu) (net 1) (status 20))
 (segment (start 124.05 68.11) (end 124.05 68.7975) (width 0.5) (layer F.Cu) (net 1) (status 10))
 (segment (start 120.760001 62.230001) (end 120.4 61.87) (width 0.5) (layer B.Cu) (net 1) (status 30))
 (segment (start 123.049999 62.230001) (end 120.760001 62.230001) (width 0.5) (layer B.Cu) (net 1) (status 20))
 (segment (start 123.27 62.01) (end 123.049999 62.230001) (width 0.5) (layer B.Cu) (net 1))
 (segment (start 120.4 63.91) (end 120.27 64.04) (width 0.5) (layer B.Cu) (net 1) (status 30))
 (segment (start 120.4 61.87) (end 120.4 63.91) (width 0.5) (layer B.Cu) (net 1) (status 30))
 (segment (start 120.4595 69.088) (end 120.4595 70.7305) (width 0.5) (layer F.Cu) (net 1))
 (segment (start 120.71751 68.82999) (end 120.4595 69.088) (width 0.5) (layer F.Cu) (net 1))
 (segment (start 124.08249 68.82999) (end 120.71751 68.82999) (width 0.5) (layer F.Cu) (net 1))
 (segment (start 125.0825 69.83) (end 124.08249 68.82999) (width 0.5) (layer F.Cu) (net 1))
 (segment (start 118.91 67.15) (end 118.91 66.637) (width 0.5) (layer F.Cu) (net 1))
 (segment (start 120.58999 68.82999) (end 118.91 67.15) (width 0.5) (layer F.Cu) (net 1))
 (segment (start 120.71751 68.82999) (end 120.58999 68.82999) (width 0.5) (layer F.Cu) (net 1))
 (via (at 134.39 93.97) (size 0.5) (drill 0.3) (layers F.Cu B.Cu) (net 5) (status 30))
 (via (at 134.36 93.36) (size 0.5) (drill 0.3) (layers F.Cu B.Cu) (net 5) (status 30))
 (via (at 133.33 93.67) (size 0.8) (drill 0.4) (layers F.Cu B.Cu) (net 5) (status 30))
 (via (at 132.334 75.3872) (size 0.8) (drill 0.4) (layers F.Cu B.Cu) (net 5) (status 30))
 (segment (start 130.209989 90.274189) (end 130.209989 79.761469) (width 0.5) (layer B.Cu) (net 5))
 (segment (start 130.209989 79.761469) (end 132.334 77.637458) (width 0.5) (layer B.Cu) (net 5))
 (segment (start 132.334 77.637458) (end 132.334 75.3872) (width 0.5) (layer B.Cu) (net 5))
 (segment (start 133.5348 93.599) (end 130.209989 90.274189) (width 0.5) (layer B.Cu) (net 5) (status 10))
 (segment (start 118.919999 78.079997) (end 119.869999 79.029997) (width 0.5) (layer F.Cu) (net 5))
 (segment (start 116.96 67.19) (end 118.919999 69.149999) (width 0.5) (layer F.Cu) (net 5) (status 10))
 (segment (start 118.919999 69.149999) (end 118.919999 78.079997) (width 0.5) (layer F.Cu) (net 5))
 (segment (start 119.869999 79.029997) (end 119.869999 81.959999) (width 0.5) (layer F.Cu) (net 5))
 (segment (start 119.869999 81.959999) (end 131.57 93.66) (width 0.5) (layer F.Cu) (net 5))
 (segment (start 131.57 93.66) (end 133.32 93.66) (width 0.5) (layer F.Cu) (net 5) (status 20))
 (via (at 118.256199 79.686001) (size 0.8) (drill 0.4) (layers F.Cu B.Cu) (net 7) (status 30))
 (segment (start 118.256199 73.566199) (end 118.256199 79.686001) (width 0.5) (layer B.Cu) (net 7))
 (segment (start 116.96 72.27) (end 118.256199 73.566199) (width 0.5) (layer B.Cu) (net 7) (status 10))
 (via (at 117.16 81.99) (size 0.5) (drill 0.3) (layers F.Cu B.Cu) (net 6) (status 30))
 (via (at 119.08 81.96) (size 0.5) (drill 0.3) (layers F.Cu B.Cu) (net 6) (status 30))
 (via (at 119.08 81.39) (size 0.5) (drill 0.3) (layers F.Cu B.Cu) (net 6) (status 30))
 (via (at 117.414999 81.335001) (size 0.5) (drill 0.3) (layers F.Cu B.Cu) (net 6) (status 30))
 (via (at 118.13 81.67) (size 0.5) (drill 0.3) (layers F.Cu B.Cu) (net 6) (status 30))
 (segment (start 116.96 69.73) (end 120.777 73.547) (width 0.5) (layer B.Cu) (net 6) (status 10))
 (segment (start 120.777 79.023) (end 118.13 81.67) (width 0.5) (layer B.Cu) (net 6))
 (segment (start 120.777 73.547) (end 120.777 79.023) (width 0.5) (layer B.Cu) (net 6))
 (via (at 134.4422 75.3872) (size 0.8) (drill 0.4) (layers F.Cu B.Cu) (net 13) (status 30))
 (via (at 133.378462 89.715862) (size 0.8) (drill 0.4) (layers F.Cu B.Cu) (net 13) (status 30))
 (segment (start 134.4422 76.499798) (end 130.81 80.131998) (width 0.5) (layer B.Cu) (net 13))
 (segment (start 134.4422 75.3872) (end 134.4422 76.499798) (width 0.5) (layer B.Cu) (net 13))
 (segment (start 130.81 80.131998) (end 130.81 89.027) (width 0.5) (layer B.Cu) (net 13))
 (segment (start 131.498862 89.715862) (end 132.153138 89.715862) (width 0.5) (layer B.Cu) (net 13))
 (segment (start 130.81 89.027) (end 131.498862 89.715862) (width 0.5) (layer B.Cu) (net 13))
 (segment (start 132.153138 89.715862) (end 133.378462 89.715862) (width 0.5) (layer B.Cu) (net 13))
 (via (at 132.153138 89.715862) (size 0.8) (drill 0.4) (layers F.Cu B.Cu) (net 13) (status 30))
 (segment (start 127.7874 77.0926) (end 126.72 78.16) (width 0.5) (layer F.Cu) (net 11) (status 20))
 (segment (start 127.7874 75.3488) (end 127.7874 77.0926) (width 0.5) (layer F.Cu) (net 11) (status 10))
 (via (at 124.73 77.53) (size 0.5) (drill 0.3) (layers F.Cu B.Cu) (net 2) (status 30))
 (via (at 124.73 78.28) (size 0.5) (drill 0.3) (layers F.Cu B.Cu) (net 2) (status 30))
 (via (at 124.73 78.95) (size 0.5) (drill 0.3) (layers F.Cu B.Cu) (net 2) (status 30))
 (segment (start 125.5268 77.3532) (end 124.72 78.16) (width 0.5) (layer F.Cu) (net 2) (status 20))
 (segment (start 125.5268 75.368) (end 125.5268 77.3532) (width 0.5) (layer F.Cu) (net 2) (status 10))
 (segment (start 120.571201 74.318799) (end 120.4595 74.4305) (width 0.5) (layer F.Cu) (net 2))
 (segment (start 124.477599 74.318799) (end 120.571201 74.318799) (width 0.5) (layer F.Cu) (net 2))
 (segment (start 125.5268 75.368) (end 124.477599 74.318799) (width 0.5) (layer F.Cu) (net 2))
 (via (at 126.74972 64.046) (size 0.5) (drill 0.3) (layers F.Cu B.Cu) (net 3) (status 30))
 (via (at 124.74972 65.046) (size 0.5) (drill 0.3) (layers F.Cu B.Cu) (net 3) (status 30))
 (via (at 124.74972 63.046) (size 0.5) (drill 0.3) (layers F.Cu B.Cu) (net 3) (status 30))
 (via (at 125.74972 63.046) (size 0.5) (drill 0.3) (layers F.Cu B.Cu) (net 3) (status 30))
 (via (at 126.83 63.1) (size 0.5) (drill 0.3) (layers F.Cu B.Cu) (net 3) (status 30))
 (via (at 124.74972 64.046) (size 0.5) (drill 0.3) (layers F.Cu B.Cu) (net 3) (status 30))
 (via (at 125.7708 64.0092) (size 0.8) (drill 0.4) (layers F.Cu B.Cu) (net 3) (status 30))
 (via (at 126.74972 65.046) (size 0.5) (drill 0.3) (layers F.Cu B.Cu) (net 3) (status 30))
 (via (at 125.74972 65.046) (size 0.5) (drill 0.3) (layers F.Cu B.Cu) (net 3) (status 30))
 (segment (start 122.35 56.38) (end 128.85 56.38) (width 0.5) (layer F.Cu) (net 3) (status 30))
 (segment (start 127.040001 62.230001) (end 126.82 62.01) (width 0.5) (layer B.Cu) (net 3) (status 30))
 (segment (start 130.091999 62.230001) (end 127.040001 62.230001) (width 0.5) (layer B.Cu) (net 3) (status 20))
 (segment (start 131.632 60.69) (end 130.091999 62.230001) (width 0.5) (layer B.Cu) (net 3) (status 10))
 (segment (start 126.82 58.41) (end 126.82 62.01) (width 0.5) (layer B.Cu) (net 3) (status 20))
 (segment (start 128.85 56.38) (end 126.82 58.41) (width 0.5) (layer B.Cu) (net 3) (status 10))
 (segment (start 125.7808 63.0492) (end 126.82 62.01) (width 0.5) (layer B.Cu) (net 3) (status 30))
 (segment (start 125.7808 64.0842) (end 125.7808 63.0492) (width 0.5) (layer B.Cu) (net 3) (status 30))
 (segment (start 128.98 64.17) (end 126.82 62.01) (width 0.5) (layer B.Cu) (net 3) (status 20))
 (segment (start 130.98 64.17) (end 128.98 64.17) (width 0.5) (layer B.Cu) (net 3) (status 10))
 (segment (start 120.661 59.309) (end 118.1 61.87) (width 0.5) (layer B.Cu) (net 3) (status 20))
 (segment (start 124.119 59.309) (end 120.661 59.309) (width 0.5) (layer B.Cu) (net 3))
 (segment (start 126.82 62.01) (end 124.119 59.309) (width 0.5) (layer B.Cu) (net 3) (status 10))
 (segment (start 118.1 62.82) (end 119.32 64.04) (width 0.5) (layer B.Cu) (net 3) (status 20))
 (segment (start 118.1 61.87) (end 118.1 62.82) (width 0.5) (layer B.Cu) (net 3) (status 10))
 (segment (start 133.135003 65.869999) (end 132.330001 65.869999) (width 0.5) (layer B.Cu) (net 14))
 (segment (start 134.099999 64.905003) (end 133.135003 65.869999) (width 0.5) (layer B.Cu) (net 14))
 (segment (start 134.099999 61.778001) (end 134.099999 64.905003) (width 0.5) (layer B.Cu) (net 14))
 (segment (start 132.330001 65.869999) (end 130.98 67.22) (width 0.5) (layer B.Cu) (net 14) (status 20))
 (segment (start 135.188 60.69) (end 134.099999 61.778001) (width 0.5) (layer B.Cu) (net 14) (status 10))
 (segment (start 130.048 76.832) (end 128.72 78.16) (width 0.5) (layer F.Cu) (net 12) (status 20))
 (segment (start 130.048 75.3488) (end 130.048 76.832) (width 0.5) (layer F.Cu) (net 12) (status 10))
 (segment (start 130.58501 66.64) (end 132.85 64.37501) (width 0.5) (layer F.Cu) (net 15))
 (via (at 132.85 64.37501) (size 0.8) (drill 0.4) (layers F.Cu B.Cu) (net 15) (status 30))
 (segment (start 122.9 66.64) (end 130.58501 66.64) (width 0.5) (layer F.Cu) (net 15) (status 10))
 (via (at 122.7836 78.2066) (size 0.5) (drill 0.3) (layers F.Cu B.Cu) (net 10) (status 30))
 (segment (start 122.7836 78.2066) (end 122.7836 68.2036) (width 0.5) (layer B.Cu) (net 10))
 (segment (start 122.7836 68.2036) (end 121.22 66.64) (width 0.5) (layer B.Cu) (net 10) (status 20))
 (via (at 122.7836 68.2036) (size 0.5) (drill 0.3) (layers F.Cu B.Cu) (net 10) (status 30))
 (segment (start 123.0376 69.9499) (end 123.1575 69.83) (width 0.5) (layer F.Cu) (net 17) (status 30))
 (segment (start 123.0376 73.0188) (end 123.0376 69.9499) (width 0.5) (layer F.Cu) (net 17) (status 30))
 (segment (start 123.0376 75.8424) (end 120.72 78.16) (width 0.5) (layer F.Cu) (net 9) (status 30))
 (segment (start 123.0376 75.4188) (end 123.0376 75.8424) (width 0.5) (layer F.Cu) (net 9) (status 30))
 (segment (start 131.41 60.495) (end 131.45 60.535) (width 0.5) (layer F.Cu) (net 18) (status 30))
 (segment (start 131.41 58.52) (end 131.41 60.495) (width 0.5) (layer F.Cu) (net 18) (status 30))
 (via (at 121.33 64.13) (size 0.8) (drill 0.4) (layers F.Cu B.Cu) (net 4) (status 30))
 (segment (start 122.35 63.09) (end 121.31 64.13) (width 0.5) (layer F.Cu) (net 4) (status 20))
 (segment (start 122.35 60.88) (end 122.35 63.09) (width 0.5) (layer F.Cu) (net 4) (status 10))
 (segment (start 122.35 60.88) (end 128.85 60.88) (width 0.5) (layer F.Cu) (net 4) (status 30))
 (segment (start 128.85 58.68) (end 131.41 56.12) (width 0.5) (layer F.Cu) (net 4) (status 20))
 (segment (start 128.85 60.88) (end 128.85 58.68) (width 0.5) (layer F.Cu) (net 4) (status 10))
 (segment (start 131.41 56.12) (end 131.41 56.135) (width 0.5) (layer F.Cu) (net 4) (status 30))
 (via (at 120.21 66.67) (size 0.8) (drill 0.4) (layers F.Cu B.Cu) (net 16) (status 30))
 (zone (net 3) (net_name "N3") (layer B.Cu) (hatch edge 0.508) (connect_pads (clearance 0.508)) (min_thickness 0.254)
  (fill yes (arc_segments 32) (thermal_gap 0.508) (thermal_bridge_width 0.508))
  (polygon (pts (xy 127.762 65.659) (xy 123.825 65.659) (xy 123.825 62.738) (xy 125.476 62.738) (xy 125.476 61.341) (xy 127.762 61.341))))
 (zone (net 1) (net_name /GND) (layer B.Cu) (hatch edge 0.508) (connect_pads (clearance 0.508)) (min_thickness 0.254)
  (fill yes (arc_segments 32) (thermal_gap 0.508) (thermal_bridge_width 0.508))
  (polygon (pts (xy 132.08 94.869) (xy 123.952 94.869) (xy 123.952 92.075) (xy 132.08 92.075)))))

